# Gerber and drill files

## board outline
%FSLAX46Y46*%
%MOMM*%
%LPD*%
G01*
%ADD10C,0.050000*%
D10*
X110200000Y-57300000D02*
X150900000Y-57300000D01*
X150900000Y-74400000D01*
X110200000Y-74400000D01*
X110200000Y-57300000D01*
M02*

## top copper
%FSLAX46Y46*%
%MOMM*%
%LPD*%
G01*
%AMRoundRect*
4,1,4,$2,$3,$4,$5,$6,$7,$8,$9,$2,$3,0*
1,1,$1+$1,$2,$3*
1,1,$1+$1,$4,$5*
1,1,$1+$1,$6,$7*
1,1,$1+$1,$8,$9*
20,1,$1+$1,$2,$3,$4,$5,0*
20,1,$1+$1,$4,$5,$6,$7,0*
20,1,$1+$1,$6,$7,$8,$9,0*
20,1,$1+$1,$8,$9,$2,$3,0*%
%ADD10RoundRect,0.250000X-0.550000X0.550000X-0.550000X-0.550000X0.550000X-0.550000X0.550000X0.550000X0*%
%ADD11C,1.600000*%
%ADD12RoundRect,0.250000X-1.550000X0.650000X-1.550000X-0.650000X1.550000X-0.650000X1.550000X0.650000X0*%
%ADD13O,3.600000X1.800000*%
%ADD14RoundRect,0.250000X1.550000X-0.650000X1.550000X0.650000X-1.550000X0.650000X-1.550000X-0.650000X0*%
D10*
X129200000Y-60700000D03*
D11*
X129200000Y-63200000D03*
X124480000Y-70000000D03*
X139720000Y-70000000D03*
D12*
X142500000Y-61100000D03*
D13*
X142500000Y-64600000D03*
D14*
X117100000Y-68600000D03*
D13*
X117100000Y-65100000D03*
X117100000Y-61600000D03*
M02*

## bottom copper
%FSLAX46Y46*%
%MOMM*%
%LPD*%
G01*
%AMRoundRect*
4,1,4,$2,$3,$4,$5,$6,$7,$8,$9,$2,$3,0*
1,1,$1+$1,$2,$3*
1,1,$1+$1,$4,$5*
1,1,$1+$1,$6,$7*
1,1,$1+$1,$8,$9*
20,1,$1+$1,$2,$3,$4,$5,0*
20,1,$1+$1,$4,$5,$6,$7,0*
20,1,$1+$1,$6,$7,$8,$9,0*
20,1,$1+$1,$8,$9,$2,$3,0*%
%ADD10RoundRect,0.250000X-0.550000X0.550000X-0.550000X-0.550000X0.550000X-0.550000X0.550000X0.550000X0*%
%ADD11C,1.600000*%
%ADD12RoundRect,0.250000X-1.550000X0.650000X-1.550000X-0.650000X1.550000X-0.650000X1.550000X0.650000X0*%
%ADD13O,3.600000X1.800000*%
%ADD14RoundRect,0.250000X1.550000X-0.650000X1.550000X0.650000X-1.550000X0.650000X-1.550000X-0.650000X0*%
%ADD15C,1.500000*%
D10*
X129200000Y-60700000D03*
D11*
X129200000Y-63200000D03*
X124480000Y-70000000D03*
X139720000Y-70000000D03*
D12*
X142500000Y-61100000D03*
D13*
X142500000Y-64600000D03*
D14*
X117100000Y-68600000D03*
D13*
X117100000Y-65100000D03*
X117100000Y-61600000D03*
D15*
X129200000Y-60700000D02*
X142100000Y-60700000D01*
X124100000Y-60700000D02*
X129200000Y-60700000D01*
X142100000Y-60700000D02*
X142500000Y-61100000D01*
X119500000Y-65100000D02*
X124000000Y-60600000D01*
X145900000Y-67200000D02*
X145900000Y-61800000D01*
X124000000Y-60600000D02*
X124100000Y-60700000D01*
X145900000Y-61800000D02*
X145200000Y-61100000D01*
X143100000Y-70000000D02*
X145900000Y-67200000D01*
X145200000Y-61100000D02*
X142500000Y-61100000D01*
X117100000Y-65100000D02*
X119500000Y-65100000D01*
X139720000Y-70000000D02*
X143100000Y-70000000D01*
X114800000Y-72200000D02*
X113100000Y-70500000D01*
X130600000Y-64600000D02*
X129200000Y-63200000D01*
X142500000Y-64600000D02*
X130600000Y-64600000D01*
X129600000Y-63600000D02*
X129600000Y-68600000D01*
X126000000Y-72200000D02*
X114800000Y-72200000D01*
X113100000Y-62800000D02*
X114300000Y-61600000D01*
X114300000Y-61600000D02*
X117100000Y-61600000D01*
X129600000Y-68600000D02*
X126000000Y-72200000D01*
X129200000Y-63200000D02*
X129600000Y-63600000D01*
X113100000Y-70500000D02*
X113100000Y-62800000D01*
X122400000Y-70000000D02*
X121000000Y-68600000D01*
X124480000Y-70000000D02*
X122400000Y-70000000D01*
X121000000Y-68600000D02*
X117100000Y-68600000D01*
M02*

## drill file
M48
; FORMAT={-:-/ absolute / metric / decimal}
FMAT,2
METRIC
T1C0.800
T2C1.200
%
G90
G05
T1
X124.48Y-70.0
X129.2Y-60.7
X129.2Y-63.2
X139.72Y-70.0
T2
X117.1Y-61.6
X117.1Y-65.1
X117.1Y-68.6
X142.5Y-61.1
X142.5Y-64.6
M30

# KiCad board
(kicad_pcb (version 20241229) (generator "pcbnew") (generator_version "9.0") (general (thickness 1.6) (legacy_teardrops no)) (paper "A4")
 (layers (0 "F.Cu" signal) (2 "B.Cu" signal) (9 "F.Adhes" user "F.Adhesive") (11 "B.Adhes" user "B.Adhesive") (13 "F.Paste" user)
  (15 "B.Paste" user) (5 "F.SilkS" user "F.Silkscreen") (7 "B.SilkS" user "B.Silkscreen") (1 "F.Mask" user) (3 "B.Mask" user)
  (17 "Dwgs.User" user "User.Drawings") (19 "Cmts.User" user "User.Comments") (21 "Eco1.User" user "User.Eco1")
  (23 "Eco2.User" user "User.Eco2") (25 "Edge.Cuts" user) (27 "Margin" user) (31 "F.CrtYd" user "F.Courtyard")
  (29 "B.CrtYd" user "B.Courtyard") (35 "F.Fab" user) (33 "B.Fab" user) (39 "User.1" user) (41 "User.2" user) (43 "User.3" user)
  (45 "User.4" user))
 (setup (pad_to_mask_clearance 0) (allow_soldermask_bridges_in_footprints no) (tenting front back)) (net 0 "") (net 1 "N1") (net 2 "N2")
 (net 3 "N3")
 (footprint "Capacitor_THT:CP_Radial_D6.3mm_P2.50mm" (layer "F.Cu") (at 129.2 60.7 -90)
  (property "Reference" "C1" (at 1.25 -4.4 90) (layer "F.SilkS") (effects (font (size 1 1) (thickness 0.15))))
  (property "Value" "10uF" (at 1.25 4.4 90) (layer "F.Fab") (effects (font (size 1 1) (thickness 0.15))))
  (pad "1" thru_hole roundrect (at 0 0 270) (size 1.6 1.6) (drill 0.8) (layers "*.Cu" "*.Mask") (remove_unused_layers no)
   (roundrect_rratio 0.15625) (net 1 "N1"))
  (pad "2" thru_hole circle (at 2.5 0 270) (size 1.6 1.6) (drill 0.8) (layers "*.Cu" "*.Mask") (remove_unused_layers no) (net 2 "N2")))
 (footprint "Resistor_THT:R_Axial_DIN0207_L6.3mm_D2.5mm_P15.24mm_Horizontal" (layer "F.Cu") (at 124.48 70)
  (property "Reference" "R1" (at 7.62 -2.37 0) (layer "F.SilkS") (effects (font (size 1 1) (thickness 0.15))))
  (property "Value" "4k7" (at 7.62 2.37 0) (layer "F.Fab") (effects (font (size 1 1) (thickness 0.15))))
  (pad "1" thru_hole circle (at 0 0) (size 1.6 1.6) (drill 0.8) (layers "*.Cu" "*.Mask") (remove_unused_layers no) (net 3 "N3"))
  (pad "2" thru_hole circle (at 15.24 0) (size 1.6 1.6) (drill 0.8) (layers "*.Cu" "*.Mask") (remove_unused_layers no) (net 1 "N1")))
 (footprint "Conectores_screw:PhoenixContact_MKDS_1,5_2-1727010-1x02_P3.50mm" (layer "F.Cu") (at 145.04 61.1 -90)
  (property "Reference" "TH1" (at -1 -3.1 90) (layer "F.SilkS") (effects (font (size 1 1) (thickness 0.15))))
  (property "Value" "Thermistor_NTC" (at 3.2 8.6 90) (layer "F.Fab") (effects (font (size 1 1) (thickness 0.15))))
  (pad "1" thru_hole roundrect (at 0 2.54 270) (size 1.8 3.6) (drill 1.2) (layers "*.Cu" "*.Mask") (remove_unused_layers no)
   (roundrect_rratio 0.138889) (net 1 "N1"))
  (pad "2" thru_hole oval (at 3.5 2.54 270) (size 1.8 3.6) (drill 1.2) (layers "*.Cu" "*.Mask") (remove_unused_layers no) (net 2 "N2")))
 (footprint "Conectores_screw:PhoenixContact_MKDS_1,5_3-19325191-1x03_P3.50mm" (layer "F.Cu") (at 114.56 68.6 90)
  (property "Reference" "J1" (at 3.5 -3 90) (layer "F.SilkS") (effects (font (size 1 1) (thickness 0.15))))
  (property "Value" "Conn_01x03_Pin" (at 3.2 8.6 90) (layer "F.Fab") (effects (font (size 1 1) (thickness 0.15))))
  (pad "1" thru_hole roundrect (at 0 2.54 90) (size 1.8 3.6) (drill 1.2) (layers "*.Cu" "*.Mask") (remove_unused_layers no)
   (roundrect_rratio 0.138889) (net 3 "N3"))
  (pad "2" thru_hole oval (at 3.5 2.54 90) (size 1.8 3.6) (drill 1.2) (layers "*.Cu" "*.Mask") (remove_unused_layers no) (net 1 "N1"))
  (pad "3" thru_hole oval (at 7 2.54 90) (size 1.8 3.6) (drill 1.2) (layers "*.Cu" "*.Mask") (remove_unused_layers no) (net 2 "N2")))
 (gr_rect (start 110.2 57.3) (end 150.9 74.4) (stroke (width 0.05) (type default)) (fill no) (layer "Edge.Cuts"))
 (segment (start 129.2 60.7) (end 142.1 60.7) (width 1.5) (layer "B.Cu") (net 1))
 (segment (start 124.1 60.7) (end 129.2 60.7) (width 1.5) (layer "B.Cu") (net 1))
 (segment (start 142.1 60.7) (end 142.5 61.1) (width 1.5) (layer "B.Cu") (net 1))
 (segment (start 119.5 65.1) (end 124 60.6) (width 1.5) (layer "B.Cu") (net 1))
 (segment (start 145.9 67.2) (end 145.9 61.8) (width 1.5) (layer "B.Cu") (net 1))
 (segment (start 124 60.6) (end 124.1 60.7) (width 1.5) (layer "B.Cu") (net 1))
 (segment (start 145.9 61.8) (end 145.2 61.1) (width 1.5) (layer "B.Cu") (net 1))
 (segment (start 143.1 70) (end 145.9 67.2) (width 1.5) (layer "B.Cu") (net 1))
 (segment (start 145.2 61.1) (end 142.5 61.1) (width 1.5) (layer "B.Cu") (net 1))
 (segment (start 117.1 65.1) (end 119.5 65.1) (width 1.5) (layer "B.Cu") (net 1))
 (segment (start 139.72 70) (end 143.1 70) (width 1.5) (layer "B.Cu") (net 1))
 (segment (start 114.8 72.2) (end 113.1 70.5) (width 1.5) (layer "B.Cu") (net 2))
 (segment (start 130.6 64.6) (end 129.2 63.2) (width 1.5) (layer "B.Cu") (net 2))
 (segment (start 142.5 64.6) (end 130.6 64.6) (width 1.5) (layer "B.Cu") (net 2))
 (segment (start 129.6 63.6) (end 129.6 68.6) (width 1.5) (layer "B.Cu") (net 2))
 (segment (start 126 72.2) (end 114.8 72.2) (width 1.5) (layer "B.Cu") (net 2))
 (segment (start 113.1 62.8) (end 114.3 61.6) (width 1.5) (layer "B.Cu") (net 2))
 (segment (start 114.3 61.6) (end 117.1 61.6) (width 1.5) (layer "B.Cu") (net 2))
 (segment (start 129.6 68.6) (end 126 72.2) (width 1.5) (layer "B.Cu") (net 2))
 (segment (start 129.2 63.2) (end 129.6 63.6) (width 1.5) (layer "B.Cu") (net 2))
 (segment (start 113.1 70.5) (end 113.1 62.8) (width 1.5) (layer "B.Cu") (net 2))
 (segment (start 122.4 70) (end 121 68.6) (width 1.5) (layer "B.Cu") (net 3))
 (segment (start 124.48 70) (end 122.4 70) (width 1.5) (layer "B.Cu") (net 3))
 (segment (start 121 68.6) (end 117.1 68.6) (width 1.5) (layer "B.Cu") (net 3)))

